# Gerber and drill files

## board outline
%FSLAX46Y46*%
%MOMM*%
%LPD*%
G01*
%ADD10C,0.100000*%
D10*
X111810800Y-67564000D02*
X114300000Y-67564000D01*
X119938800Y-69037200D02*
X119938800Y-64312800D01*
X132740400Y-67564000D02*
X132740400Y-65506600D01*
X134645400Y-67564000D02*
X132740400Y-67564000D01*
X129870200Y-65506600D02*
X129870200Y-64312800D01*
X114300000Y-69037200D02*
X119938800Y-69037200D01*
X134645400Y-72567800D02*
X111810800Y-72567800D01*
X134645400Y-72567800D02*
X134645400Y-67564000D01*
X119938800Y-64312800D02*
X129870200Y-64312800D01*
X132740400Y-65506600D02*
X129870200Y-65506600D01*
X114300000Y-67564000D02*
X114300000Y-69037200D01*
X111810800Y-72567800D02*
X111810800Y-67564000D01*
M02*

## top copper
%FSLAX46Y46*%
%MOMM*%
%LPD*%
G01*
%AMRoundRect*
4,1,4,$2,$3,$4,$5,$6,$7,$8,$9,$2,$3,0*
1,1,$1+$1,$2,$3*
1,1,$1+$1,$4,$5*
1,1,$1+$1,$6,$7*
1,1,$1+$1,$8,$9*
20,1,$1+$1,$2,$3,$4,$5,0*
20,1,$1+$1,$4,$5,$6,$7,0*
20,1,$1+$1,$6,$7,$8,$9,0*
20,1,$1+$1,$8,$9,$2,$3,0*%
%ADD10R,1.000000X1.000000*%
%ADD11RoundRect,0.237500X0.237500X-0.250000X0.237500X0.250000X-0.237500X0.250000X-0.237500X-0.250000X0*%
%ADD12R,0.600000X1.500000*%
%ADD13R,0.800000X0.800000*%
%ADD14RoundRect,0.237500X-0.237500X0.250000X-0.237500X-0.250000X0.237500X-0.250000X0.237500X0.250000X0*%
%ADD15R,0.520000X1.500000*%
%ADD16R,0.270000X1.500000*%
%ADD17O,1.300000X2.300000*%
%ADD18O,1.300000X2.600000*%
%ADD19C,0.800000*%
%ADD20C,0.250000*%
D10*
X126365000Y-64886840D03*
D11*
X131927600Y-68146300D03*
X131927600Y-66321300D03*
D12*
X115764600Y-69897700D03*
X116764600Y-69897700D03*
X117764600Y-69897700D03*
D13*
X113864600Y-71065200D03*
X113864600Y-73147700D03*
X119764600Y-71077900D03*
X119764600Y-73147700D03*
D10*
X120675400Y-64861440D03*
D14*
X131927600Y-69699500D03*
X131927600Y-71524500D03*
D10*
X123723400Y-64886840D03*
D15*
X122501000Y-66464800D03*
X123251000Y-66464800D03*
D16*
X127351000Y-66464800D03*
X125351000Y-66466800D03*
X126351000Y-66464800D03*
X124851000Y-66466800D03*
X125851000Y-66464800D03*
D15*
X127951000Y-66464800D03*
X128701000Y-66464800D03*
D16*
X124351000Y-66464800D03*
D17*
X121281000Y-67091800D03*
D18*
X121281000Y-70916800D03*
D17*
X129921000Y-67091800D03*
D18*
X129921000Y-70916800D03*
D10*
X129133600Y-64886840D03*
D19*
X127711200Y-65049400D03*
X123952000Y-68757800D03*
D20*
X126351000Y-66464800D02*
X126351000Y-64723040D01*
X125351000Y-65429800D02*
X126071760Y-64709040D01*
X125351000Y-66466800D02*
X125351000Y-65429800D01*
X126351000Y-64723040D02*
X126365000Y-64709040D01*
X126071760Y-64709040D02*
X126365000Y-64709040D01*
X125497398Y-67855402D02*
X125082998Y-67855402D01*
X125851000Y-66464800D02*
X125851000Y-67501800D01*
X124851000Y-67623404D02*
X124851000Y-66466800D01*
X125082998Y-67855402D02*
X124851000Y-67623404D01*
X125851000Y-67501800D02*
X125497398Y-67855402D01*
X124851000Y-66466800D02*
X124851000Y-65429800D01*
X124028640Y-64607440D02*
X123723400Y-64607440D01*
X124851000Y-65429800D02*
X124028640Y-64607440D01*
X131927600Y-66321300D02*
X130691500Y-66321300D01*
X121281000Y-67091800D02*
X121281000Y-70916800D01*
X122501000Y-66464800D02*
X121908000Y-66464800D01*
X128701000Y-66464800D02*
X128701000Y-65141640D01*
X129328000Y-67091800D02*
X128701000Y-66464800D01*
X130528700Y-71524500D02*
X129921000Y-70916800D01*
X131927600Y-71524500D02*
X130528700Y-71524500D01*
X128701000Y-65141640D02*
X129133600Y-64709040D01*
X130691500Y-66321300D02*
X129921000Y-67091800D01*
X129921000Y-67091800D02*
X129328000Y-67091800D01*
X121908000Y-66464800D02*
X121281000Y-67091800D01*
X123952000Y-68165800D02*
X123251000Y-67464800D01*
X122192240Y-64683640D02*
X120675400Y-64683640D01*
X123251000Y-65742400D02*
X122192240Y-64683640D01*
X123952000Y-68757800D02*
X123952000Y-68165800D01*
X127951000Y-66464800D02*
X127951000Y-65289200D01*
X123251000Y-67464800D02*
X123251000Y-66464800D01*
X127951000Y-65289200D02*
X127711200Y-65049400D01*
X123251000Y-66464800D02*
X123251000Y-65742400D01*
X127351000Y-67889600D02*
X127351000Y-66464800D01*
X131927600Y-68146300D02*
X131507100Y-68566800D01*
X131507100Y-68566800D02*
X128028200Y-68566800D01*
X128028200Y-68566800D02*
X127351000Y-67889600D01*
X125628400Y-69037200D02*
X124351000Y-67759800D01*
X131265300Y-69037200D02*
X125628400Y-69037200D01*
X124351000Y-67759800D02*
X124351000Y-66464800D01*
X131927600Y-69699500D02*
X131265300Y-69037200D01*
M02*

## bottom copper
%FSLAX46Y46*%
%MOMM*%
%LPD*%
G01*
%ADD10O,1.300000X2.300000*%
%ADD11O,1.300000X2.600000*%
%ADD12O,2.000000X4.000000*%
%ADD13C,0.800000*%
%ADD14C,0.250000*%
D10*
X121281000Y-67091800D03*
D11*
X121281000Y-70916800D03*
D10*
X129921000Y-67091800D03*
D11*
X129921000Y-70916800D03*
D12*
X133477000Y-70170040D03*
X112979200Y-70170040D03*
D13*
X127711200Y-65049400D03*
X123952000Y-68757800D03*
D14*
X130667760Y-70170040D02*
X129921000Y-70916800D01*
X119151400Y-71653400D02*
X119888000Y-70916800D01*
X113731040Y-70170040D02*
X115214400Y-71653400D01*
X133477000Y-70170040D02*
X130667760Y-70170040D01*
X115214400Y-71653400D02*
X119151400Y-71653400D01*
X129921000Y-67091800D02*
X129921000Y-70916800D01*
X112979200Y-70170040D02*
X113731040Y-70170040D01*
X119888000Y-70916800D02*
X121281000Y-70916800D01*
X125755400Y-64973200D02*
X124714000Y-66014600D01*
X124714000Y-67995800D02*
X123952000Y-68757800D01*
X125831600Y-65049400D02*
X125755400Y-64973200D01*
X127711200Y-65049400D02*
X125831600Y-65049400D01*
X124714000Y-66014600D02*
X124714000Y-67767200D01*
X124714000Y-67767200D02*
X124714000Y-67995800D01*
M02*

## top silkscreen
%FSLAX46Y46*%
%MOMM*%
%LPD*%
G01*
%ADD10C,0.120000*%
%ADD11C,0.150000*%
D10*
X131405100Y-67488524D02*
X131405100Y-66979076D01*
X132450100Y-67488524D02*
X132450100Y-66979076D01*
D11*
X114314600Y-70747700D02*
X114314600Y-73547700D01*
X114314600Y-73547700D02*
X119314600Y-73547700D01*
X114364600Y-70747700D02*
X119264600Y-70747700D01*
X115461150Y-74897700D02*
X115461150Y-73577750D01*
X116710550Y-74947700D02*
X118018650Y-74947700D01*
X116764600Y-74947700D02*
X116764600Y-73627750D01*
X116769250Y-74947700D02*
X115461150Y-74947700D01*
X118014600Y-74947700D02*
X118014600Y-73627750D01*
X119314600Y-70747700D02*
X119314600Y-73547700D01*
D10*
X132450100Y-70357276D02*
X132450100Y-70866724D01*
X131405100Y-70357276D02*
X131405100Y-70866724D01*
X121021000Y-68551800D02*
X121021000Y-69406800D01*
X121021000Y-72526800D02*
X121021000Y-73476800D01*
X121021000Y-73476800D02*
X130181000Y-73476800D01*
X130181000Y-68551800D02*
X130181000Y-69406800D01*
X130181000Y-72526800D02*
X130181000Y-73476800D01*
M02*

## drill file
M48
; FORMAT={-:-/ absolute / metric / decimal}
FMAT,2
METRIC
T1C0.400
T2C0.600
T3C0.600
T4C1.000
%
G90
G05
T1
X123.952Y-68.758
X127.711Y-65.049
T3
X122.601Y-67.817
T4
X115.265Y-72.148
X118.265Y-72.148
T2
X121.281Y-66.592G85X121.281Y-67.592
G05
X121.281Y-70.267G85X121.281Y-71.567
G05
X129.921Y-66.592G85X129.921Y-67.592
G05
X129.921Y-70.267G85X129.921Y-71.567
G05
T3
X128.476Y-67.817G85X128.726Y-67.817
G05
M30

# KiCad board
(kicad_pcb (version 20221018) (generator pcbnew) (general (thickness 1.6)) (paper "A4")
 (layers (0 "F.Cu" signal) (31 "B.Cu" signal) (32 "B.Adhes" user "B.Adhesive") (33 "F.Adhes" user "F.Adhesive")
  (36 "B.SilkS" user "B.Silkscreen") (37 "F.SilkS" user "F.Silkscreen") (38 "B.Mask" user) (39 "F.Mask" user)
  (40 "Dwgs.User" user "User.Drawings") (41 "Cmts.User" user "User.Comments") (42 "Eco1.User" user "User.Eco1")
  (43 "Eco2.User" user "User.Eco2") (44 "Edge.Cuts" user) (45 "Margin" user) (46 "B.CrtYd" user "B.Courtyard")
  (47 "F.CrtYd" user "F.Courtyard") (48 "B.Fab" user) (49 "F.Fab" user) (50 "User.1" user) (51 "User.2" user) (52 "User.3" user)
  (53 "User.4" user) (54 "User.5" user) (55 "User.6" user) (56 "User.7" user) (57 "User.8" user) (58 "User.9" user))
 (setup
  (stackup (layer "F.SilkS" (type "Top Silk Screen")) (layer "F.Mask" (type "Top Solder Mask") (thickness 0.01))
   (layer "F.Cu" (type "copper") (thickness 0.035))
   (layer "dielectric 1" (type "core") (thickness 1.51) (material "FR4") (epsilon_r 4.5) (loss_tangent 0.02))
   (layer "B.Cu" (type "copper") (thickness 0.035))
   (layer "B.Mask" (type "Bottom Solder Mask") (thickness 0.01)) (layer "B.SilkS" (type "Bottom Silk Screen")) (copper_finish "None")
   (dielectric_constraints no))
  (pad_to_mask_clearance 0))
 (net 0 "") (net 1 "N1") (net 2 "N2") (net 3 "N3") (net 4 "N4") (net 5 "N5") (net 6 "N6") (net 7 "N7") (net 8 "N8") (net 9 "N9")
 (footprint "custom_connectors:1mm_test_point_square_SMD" (layer "F.Cu") (at 126.365 64.897)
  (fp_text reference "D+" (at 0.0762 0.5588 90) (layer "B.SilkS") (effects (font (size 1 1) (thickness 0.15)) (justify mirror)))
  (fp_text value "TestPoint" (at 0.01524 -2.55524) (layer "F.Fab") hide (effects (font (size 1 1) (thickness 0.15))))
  (pad "1" smd rect (at 0 -0.01016) (size 1 1) (layers "F.Cu" "F.Paste" "F.Mask") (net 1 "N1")))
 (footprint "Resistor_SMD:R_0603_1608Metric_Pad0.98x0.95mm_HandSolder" (layer "F.Cu") (at 131.9276 67.2338 90)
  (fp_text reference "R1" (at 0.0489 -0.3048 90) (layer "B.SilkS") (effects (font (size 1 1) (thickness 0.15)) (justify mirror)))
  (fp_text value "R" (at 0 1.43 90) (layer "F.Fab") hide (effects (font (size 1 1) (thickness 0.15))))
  (fp_line (start -0.254724 -0.5225) (end 0.254724 -0.5225) (stroke (width 0.12) (type solid)) (layer "F.SilkS"))
  (fp_line (start -0.254724 0.5225) (end 0.254724 0.5225) (stroke (width 0.12) (type solid)) (layer "F.SilkS"))
  (pad "1" smd roundrect (at -0.9125 0 90) (size 0.975 0.95) (layers "F.Cu" "F.Paste" "F.Mask") (roundrect_rratio 0.25) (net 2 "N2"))
  (pad "2" smd roundrect (at 0.9125 0 90) (size 0.975 0.95) (layers "F.Cu" "F.Paste" "F.Mask") (roundrect_rratio 0.25) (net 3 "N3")))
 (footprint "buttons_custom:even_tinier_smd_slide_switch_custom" (layer "F.Cu") (at 116.7646 70.7477)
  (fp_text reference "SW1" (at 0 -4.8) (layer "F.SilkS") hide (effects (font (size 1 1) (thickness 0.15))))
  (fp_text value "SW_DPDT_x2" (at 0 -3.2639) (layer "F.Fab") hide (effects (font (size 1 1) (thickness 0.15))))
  (fp_line (start -2.45 0) (end -2.45 2.8) (stroke (width 0.15) (type solid)) (layer "F.SilkS"))
  (fp_line (start -2.45 2.8) (end 2.55 2.8) (stroke (width 0.15) (type solid)) (layer "F.SilkS"))
  (fp_line (start -2.4 0) (end 2.5 0) (stroke (width 0.15) (type solid)) (layer "F.SilkS"))
  (fp_line (start -1.30345 4.15) (end -1.30345 2.83005) (stroke (width 0.15) (type solid)) (layer "F.SilkS"))
  (fp_line (start -0.05405 4.2) (end 1.25405 4.2) (stroke (width 0.15) (type solid)) (layer "F.SilkS"))
  (fp_line (start 0 4.2) (end 0 2.88005) (stroke (width 0.15) (type solid)) (layer "F.SilkS"))
  (fp_line (start 0.00465 4.2) (end -1.30345 4.2) (stroke (width 0.15) (type solid)) (layer "F.SilkS"))
  (fp_line (start 1.25 4.2) (end 1.25 2.88005) (stroke (width 0.15) (type solid)) (layer "F.SilkS"))
  (fp_line (start 2.55 0) (end 2.55 2.8) (stroke (width 0.15) (type solid)) (layer "F.SilkS"))
  (pad "" np_thru_hole circle (at -1.5 1.4) (size 1 1) (drill 1) (layers "F&B.Cu" "*.Mask"))
  (pad "" np_thru_hole circle (at 1.5 1.4) (size 1 1) (drill 1) (layers "F&B.Cu" "*.Mask"))
  (pad "1" smd rect (at -1 -0.85) (size 0.6 1.5) (layers "F.Cu" "F.Paste" "F.Mask") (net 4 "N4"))
  (pad "2" smd rect (at 0 -0.85) (size 0.6 1.5) (layers "F.Cu" "F.Paste" "F.Mask") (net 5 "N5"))
  (pad "3" smd rect (at 1 -0.85) (size 0.6 1.5) (layers "F.Cu" "F.Paste" "F.Mask") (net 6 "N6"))
  (pad "4" smd rect (at -2.9 0.3175 90) (size 0.8 0.8) (layers "F.Cu" "F.Paste" "F.Mask"))
  (pad "4" smd rect (at -2.9 2.4 90) (size 0.8 0.8) (layers "F.Cu" "F.Paste" "F.Mask"))
  (pad "4" smd rect (at 3 0.3302 90) (size 0.8 0.8) (layers "F.Cu" "F.Paste" "F.Mask"))
  (pad "4" smd rect (at 3 2.4 90) (size 0.8 0.8) (layers "F.Cu" "F.Paste" "F.Mask")))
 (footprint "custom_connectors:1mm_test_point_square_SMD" (layer "F.Cu") (at 120.6754 64.8716)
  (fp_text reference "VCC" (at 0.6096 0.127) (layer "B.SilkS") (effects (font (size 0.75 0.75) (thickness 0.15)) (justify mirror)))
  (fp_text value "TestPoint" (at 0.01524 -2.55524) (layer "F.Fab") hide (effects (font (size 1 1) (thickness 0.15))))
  (pad "1" smd rect (at 0 -0.01016) (size 1 1) (layers "F.Cu" "F.Paste" "F.Mask") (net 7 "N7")))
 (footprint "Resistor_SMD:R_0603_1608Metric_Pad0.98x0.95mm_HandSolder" (layer "F.Cu") (at 131.9276 70.612 -90)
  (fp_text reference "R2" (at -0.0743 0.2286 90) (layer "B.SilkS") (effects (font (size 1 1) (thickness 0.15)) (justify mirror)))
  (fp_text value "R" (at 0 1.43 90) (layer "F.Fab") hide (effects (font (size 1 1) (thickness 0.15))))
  (fp_line (start -0.254724 -0.5225) (end 0.254724 -0.5225) (stroke (width 0.12) (type solid)) (layer "F.SilkS"))
  (fp_line (start -0.254724 0.5225) (end 0.254724 0.5225) (stroke (width 0.12) (type solid)) (layer "F.SilkS"))
  (pad "1" smd roundrect (at -0.9125 0 270) (size 0.975 0.95) (layers "F.Cu" "F.Paste" "F.Mask") (roundrect_rratio 0.25) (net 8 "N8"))
  (pad "2" smd roundrect (at 0.9125 0 270) (size 0.975 0.95) (layers "F.Cu" "F.Paste" "F.Mask") (roundrect_rratio 0.25) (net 3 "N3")))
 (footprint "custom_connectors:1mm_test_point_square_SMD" (layer "F.Cu") (at 123.7234 64.897)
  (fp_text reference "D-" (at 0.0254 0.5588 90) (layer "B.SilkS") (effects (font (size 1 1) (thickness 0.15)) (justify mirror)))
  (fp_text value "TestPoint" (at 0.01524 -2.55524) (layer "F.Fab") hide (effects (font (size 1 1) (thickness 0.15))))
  (pad "1" smd rect (at 0 -0.01016) (size 1 1) (layers "F.Cu" "F.Paste" "F.Mask") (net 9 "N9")))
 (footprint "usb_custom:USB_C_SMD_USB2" (layer "F.Cu") (at 125.601 69.7668)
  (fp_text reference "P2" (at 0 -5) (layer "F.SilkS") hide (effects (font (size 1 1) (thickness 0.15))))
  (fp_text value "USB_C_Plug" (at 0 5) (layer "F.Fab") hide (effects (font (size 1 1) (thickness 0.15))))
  (fp_line (start -4.58 -1.215) (end -4.58 -0.36) (stroke (width 0.12) (type solid)) (layer "F.SilkS"))
  (fp_line (start -4.58 2.76) (end -4.58 3.71) (stroke (width 0.12) (type solid)) (layer "F.SilkS"))
  (fp_line (start -4.58 3.71) (end 4.58 3.71) (stroke (width 0.12) (type solid)) (layer "F.SilkS"))
  (fp_line (start 4.58 -1.215) (end 4.58 -0.36) (stroke (width 0.12) (type solid)) (layer "F.SilkS"))
  (fp_line (start 4.58 2.76) (end 4.58 3.71) (stroke (width 0.12) (type solid)) (layer "F.SilkS"))
  (pad "" np_thru_hole circle (at -3 -1.95) (size 0.6 0.6) (drill 0.6) (layers "F&B.Cu" "*.Mask"))
  (pad "" np_thru_hole oval (at 3 -1.95) (size 0.85 0.6) (drill oval 0.85 0.6) (layers "F&B.Cu" "*.Mask"))
  (pad "A1" smd rect (at -3.1 -3.302) (size 0.52 1.5) (layers "F.Cu" "F.Paste" "F.Mask") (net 3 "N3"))
  (pad "A4" smd rect (at -2.35 -3.302) (size 0.52 1.5) (layers "F.Cu" "F.Paste" "F.Mask") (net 7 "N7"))
  (pad "A5" smd rect (at 1.75 -3.302) (size 0.27 1.5) (layers "F.Cu" "F.Paste" "F.Mask") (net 2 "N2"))
  (pad "A6" smd rect (at -0.25 -3.3) (size 0.27 1.5) (layers "F.Cu" "F.Paste" "F.Mask") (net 1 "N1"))
  (pad "A6" smd rect (at 0.75 -3.302) (size 0.27 1.5) (layers "F.Cu" "F.Paste" "F.Mask") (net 1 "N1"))
  (pad "A7" smd rect (at -0.75 -3.3) (size 0.27 1.5) (layers "F.Cu" "F.Paste" "F.Mask") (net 9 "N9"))
  (pad "A7" smd rect (at 0.25 -3.302) (size 0.27 1.5) (layers "F.Cu" "F.Paste" "F.Mask") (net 9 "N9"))
  (pad "A9" smd rect (at 2.35 -3.302) (size 0.52 1.5) (layers "F.Cu" "F.Paste" "F.Mask") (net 7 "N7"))
  (pad "A12" smd rect (at 3.1 -3.302) (size 0.52 1.5) (layers "F.Cu" "F.Paste" "F.Mask") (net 3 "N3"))
  (pad "B5" smd rect (at -1.25 -3.302) (size 0.27 1.5) (layers "F.Cu" "F.Paste" "F.Mask") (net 8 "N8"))
  (pad "S1" thru_hole oval (at -4.32 -2.675) (size 1.3 2.3) (drill oval 0.6 1.6) (layers "*.Cu" "*.Mask") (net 3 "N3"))
  (pad "S1" thru_hole oval (at -4.32 1.15) (size 1.3 2.6) (drill oval 0.6 1.9) (layers "*.Cu" "*.Mask") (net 3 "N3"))
  (pad "S1" thru_hole oval (at 4.32 -2.675) (size 1.3 2.3) (drill oval 0.6 1.6) (layers "*.Cu" "*.Mask") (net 3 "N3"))
  (pad "S1" thru_hole oval (at 4.32 1.15) (size 1.3 2.6) (drill oval 0.6 1.9) (layers "*.Cu" "*.Mask") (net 3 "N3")))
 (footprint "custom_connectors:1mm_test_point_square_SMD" (layer "F.Cu") (at 129.1336 64.897)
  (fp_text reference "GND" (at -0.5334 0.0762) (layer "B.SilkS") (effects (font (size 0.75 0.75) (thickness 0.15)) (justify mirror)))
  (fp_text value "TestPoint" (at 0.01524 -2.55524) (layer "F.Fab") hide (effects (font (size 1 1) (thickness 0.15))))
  (pad "1" smd rect (at 0 -0.01016) (size 1 1) (layers "F.Cu" "F.Paste" "F.Mask") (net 3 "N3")))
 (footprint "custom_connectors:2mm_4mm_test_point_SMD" (layer "B.Cu") (at 133.477 70.1802 180)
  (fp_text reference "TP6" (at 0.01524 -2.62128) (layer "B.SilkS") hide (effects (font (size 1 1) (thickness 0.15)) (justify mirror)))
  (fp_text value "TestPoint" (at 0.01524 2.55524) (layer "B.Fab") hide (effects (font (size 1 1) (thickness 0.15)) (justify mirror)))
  (pad "1" smd oval (at 0 0.01016 180) (size 2 4) (layers "B.Cu" "B.Paste" "B.Mask") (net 3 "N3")))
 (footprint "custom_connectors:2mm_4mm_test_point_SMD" (layer "B.Cu") (at 112.9792 70.1802 180)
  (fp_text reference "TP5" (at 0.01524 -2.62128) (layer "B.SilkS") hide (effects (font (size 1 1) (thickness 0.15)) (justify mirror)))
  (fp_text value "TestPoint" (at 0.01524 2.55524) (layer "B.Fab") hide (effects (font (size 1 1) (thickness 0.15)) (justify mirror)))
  (pad "1" smd oval (at 0 0.01016 180) (size 2 4) (layers "B.Cu" "B.Paste" "B.Mask") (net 3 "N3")))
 (gr_line (start 111.8108 67.564) (end 114.3 67.564) (stroke (width 0.1) (type default)) (layer "Edge.Cuts"))
 (gr_line (start 119.9388 69.0372) (end 119.9388 64.3128) (stroke (width 0.1) (type default)) (layer "Edge.Cuts"))
 (gr_line (start 132.7404 67.564) (end 132.7404 65.5066) (stroke (width 0.1) (type default)) (layer "Edge.Cuts"))
 (gr_line (start 134.6454 67.564) (end 132.7404 67.564) (stroke (width 0.1) (type default)) (layer "Edge.Cuts"))
 (gr_line (start 129.8702 65.5066) (end 129.8702 64.3128) (stroke (width 0.1) (type default)) (layer "Edge.Cuts"))
 (gr_line (start 114.3 69.0372) (end 119.9388 69.0372) (stroke (width 0.1) (type default)) (layer "Edge.Cuts"))
 (gr_line (start 134.6454 72.5678) (end 111.8108 72.5678) (stroke (width 0.1) (type default)) (layer "Edge.Cuts"))
 (gr_line (start 134.6454 72.5678) (end 134.6454 67.564) (stroke (width 0.1) (type default)) (layer "Edge.Cuts"))
 (gr_line (start 119.9388 64.3128) (end 129.8702 64.3128) (stroke (width 0.1) (type default)) (layer "Edge.Cuts"))
 (gr_line (start 132.7404 65.5066) (end 129.8702 65.5066) (stroke (width 0.1) (type default)) (layer "Edge.Cuts"))
 (gr_line (start 114.3 67.564) (end 114.3 69.0372) (stroke (width 0.1) (type default)) (layer "Edge.Cuts"))
 (gr_line (start 111.8108 72.5678) (end 111.8108 67.564) (stroke (width 0.1) (type default)) (layer "Edge.Cuts"))
 (segment (start 126.351 66.4648) (end 126.351 64.72304) (width 0.25) (layer "F.Cu") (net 1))
 (segment (start 125.351 65.4298) (end 126.07176 64.70904) (width 0.25) (layer "F.Cu") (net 1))
 (segment (start 125.351 66.4668) (end 125.351 65.4298) (width 0.25) (layer "F.Cu") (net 1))
 (segment (start 126.351 64.72304) (end 126.365 64.70904) (width 0.25) (layer "F.Cu") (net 1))
 (segment (start 126.07176 64.70904) (end 126.365 64.70904) (width 0.25) (layer "F.Cu") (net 1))
 (segment (start 125.497398 67.855402) (end 125.082998 67.855402) (width 0.25) (layer "F.Cu") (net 9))
 (segment (start 125.851 66.4648) (end 125.851 67.5018) (width 0.25) (layer "F.Cu") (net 9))
 (segment (start 124.851 67.623404) (end 124.851 66.4668) (width 0.25) (layer "F.Cu") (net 9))
 (segment (start 125.082998 67.855402) (end 124.851 67.623404) (width 0.25) (layer "F.Cu") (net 9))
 (segment (start 125.851 67.5018) (end 125.497398 67.855402) (width 0.25) (layer "F.Cu") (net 9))
 (segment (start 124.851 66.4668) (end 124.851 65.4298) (width 0.25) (layer "F.Cu") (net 9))
 (segment (start 124.02864 64.60744) (end 123.7234 64.60744) (width 0.25) (layer "F.Cu") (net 9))
 (segment (start 124.851 65.4298) (end 124.02864 64.60744) (width 0.25) (layer "F.Cu") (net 9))
 (segment (start 131.9276 66.3213) (end 130.6915 66.3213) (width 0.25) (layer "F.Cu") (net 3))
 (segment (start 121.281 67.0918) (end 121.281 70.9168) (width 0.25) (layer "F.Cu") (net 3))
 (segment (start 122.501 66.4648) (end 121.908 66.4648) (width 0.25) (layer "F.Cu") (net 3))
 (segment (start 128.701 66.4648) (end 128.701 65.14164) (width 0.25) (layer "F.Cu") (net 3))
 (segment (start 129.328 67.0918) (end 128.701 66.4648) (width 0.25) (layer "F.Cu") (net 3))
 (segment (start 130.5287 71.5245) (end 129.921 70.9168) (width 0.25) (layer "F.Cu") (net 3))
 (segment (start 131.9276 71.5245) (end 130.5287 71.5245) (width 0.25) (layer "F.Cu") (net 3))
 (segment (start 128.701 65.14164) (end 129.1336 64.70904) (width 0.25) (layer "F.Cu") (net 3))
 (segment (start 130.6915 66.3213) (end 129.921 67.0918) (width 0.25) (layer "F.Cu") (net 3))
 (segment (start 129.921 67.0918) (end 129.328 67.0918) (width 0.25) (layer "F.Cu") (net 3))
 (segment (start 121.908 66.4648) (end 121.281 67.0918) (width 0.25) (layer "F.Cu") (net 3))
 (segment (start 130.66776 70.17004) (end 129.921 70.9168) (width 0.25) (layer "B.Cu") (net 3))
 (segment (start 119.1514 71.6534) (end 119.888 70.9168) (width 0.25) (layer "B.Cu") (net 3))
 (segment (start 113.73104 70.17004) (end 115.2144 71.6534) (width 0.25) (layer "B.Cu") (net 3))
 (segment (start 133.477 70.17004) (end 130.66776 70.17004) (width 0.25) (layer "B.Cu") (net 3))
 (segment (start 115.2144 71.6534) (end 119.1514 71.6534) (width 0.25) (layer "B.Cu") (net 3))
 (segment (start 129.921 67.0918) (end 129.921 70.9168) (width 0.25) (layer "B.Cu") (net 3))
 (segment (start 112.9792 70.17004) (end 113.73104 70.17004) (width 0.25) (layer "B.Cu") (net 3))
 (segment (start 119.888 70.9168) (end 121.281 70.9168) (width 0.25) (layer "B.Cu") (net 3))
 (segment (start 123.952 68.1658) (end 123.251 67.4648) (width 0.25) (layer "F.Cu") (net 7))
 (segment (start 122.19224 64.68364) (end 120.6754 64.68364) (width 0.25) (layer "F.Cu") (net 7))
 (segment (start 123.251 65.7424) (end 122.19224 64.68364) (width 0.25) (layer "F.Cu") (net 7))
 (segment (start 123.952 68.7578) (end 123.952 68.1658) (width 0.25) (layer "F.Cu") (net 7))
 (segment (start 127.951 66.4648) (end 127.951 65.2892) (width 0.25) (layer "F.Cu") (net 7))
 (segment (start 123.251 67.4648) (end 123.251 66.4648) (width 0.25) (layer "F.Cu") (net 7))
 (segment (start 127.951 65.2892) (end 127.7112 65.0494) (width 0.25) (layer "F.Cu") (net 7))
 (segment (start 123.251 66.4648) (end 123.251 65.7424) (width 0.25) (layer "F.Cu") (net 7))
 (via (at 127.7112 65.0494) (size 0.8) (drill 0.4) (layers "F.Cu" "B.Cu") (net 7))
 (via (at 123.952 68.7578) (size 0.8) (drill 0.4) (layers "F.Cu" "B.Cu") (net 7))
 (segment (start 125.7554 64.9732) (end 124.714 66.0146) (width 0.25) (layer "B.Cu") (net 7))
 (segment (start 124.714 67.9958) (end 123.952 68.7578) (width 0.25) (layer "B.Cu") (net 7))
 (segment (start 125.8316 65.0494) (end 125.7554 64.9732) (width 0.25) (layer "B.Cu") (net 7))
 (segment (start 127.7112 65.0494) (end 125.8316 65.0494) (width 0.25) (layer "B.Cu") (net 7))
 (segment (start 124.714 66.0146) (end 124.714 67.7672) (width 0.25) (layer "B.Cu") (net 7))
 (segment (start 124.714 67.7672) (end 124.714 67.9958) (width 0.25) (layer "B.Cu") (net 7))
 (segment (start 127.351 67.8896) (end 127.351 66.4648) (width 0.25) (layer "F.Cu") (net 2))
 (segment (start 131.9276 68.1463) (end 131.5071 68.5668) (width 0.25) (layer "F.Cu") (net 2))
 (segment (start 131.5071 68.5668) (end 128.0282 68.5668) (width 0.25) (layer "F.Cu") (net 2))
 (segment (start 128.0282 68.5668) (end 127.351 67.8896) (width 0.25) (layer "F.Cu") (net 2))
 (segment (start 125.6284 69.0372) (end 124.351 67.7598) (width 0.25) (layer "F.Cu") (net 8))
 (segment (start 131.2653 69.0372) (end 125.6284 69.0372) (width 0.25) (layer "F.Cu") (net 8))
 (segment (start 124.351 67.7598) (end 124.351 66.4648) (width 0.25) (layer "F.Cu") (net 8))
 (segment (start 131.9276 69.6995) (end 131.2653 69.0372) (width 0.25) (layer "F.Cu") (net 8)))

